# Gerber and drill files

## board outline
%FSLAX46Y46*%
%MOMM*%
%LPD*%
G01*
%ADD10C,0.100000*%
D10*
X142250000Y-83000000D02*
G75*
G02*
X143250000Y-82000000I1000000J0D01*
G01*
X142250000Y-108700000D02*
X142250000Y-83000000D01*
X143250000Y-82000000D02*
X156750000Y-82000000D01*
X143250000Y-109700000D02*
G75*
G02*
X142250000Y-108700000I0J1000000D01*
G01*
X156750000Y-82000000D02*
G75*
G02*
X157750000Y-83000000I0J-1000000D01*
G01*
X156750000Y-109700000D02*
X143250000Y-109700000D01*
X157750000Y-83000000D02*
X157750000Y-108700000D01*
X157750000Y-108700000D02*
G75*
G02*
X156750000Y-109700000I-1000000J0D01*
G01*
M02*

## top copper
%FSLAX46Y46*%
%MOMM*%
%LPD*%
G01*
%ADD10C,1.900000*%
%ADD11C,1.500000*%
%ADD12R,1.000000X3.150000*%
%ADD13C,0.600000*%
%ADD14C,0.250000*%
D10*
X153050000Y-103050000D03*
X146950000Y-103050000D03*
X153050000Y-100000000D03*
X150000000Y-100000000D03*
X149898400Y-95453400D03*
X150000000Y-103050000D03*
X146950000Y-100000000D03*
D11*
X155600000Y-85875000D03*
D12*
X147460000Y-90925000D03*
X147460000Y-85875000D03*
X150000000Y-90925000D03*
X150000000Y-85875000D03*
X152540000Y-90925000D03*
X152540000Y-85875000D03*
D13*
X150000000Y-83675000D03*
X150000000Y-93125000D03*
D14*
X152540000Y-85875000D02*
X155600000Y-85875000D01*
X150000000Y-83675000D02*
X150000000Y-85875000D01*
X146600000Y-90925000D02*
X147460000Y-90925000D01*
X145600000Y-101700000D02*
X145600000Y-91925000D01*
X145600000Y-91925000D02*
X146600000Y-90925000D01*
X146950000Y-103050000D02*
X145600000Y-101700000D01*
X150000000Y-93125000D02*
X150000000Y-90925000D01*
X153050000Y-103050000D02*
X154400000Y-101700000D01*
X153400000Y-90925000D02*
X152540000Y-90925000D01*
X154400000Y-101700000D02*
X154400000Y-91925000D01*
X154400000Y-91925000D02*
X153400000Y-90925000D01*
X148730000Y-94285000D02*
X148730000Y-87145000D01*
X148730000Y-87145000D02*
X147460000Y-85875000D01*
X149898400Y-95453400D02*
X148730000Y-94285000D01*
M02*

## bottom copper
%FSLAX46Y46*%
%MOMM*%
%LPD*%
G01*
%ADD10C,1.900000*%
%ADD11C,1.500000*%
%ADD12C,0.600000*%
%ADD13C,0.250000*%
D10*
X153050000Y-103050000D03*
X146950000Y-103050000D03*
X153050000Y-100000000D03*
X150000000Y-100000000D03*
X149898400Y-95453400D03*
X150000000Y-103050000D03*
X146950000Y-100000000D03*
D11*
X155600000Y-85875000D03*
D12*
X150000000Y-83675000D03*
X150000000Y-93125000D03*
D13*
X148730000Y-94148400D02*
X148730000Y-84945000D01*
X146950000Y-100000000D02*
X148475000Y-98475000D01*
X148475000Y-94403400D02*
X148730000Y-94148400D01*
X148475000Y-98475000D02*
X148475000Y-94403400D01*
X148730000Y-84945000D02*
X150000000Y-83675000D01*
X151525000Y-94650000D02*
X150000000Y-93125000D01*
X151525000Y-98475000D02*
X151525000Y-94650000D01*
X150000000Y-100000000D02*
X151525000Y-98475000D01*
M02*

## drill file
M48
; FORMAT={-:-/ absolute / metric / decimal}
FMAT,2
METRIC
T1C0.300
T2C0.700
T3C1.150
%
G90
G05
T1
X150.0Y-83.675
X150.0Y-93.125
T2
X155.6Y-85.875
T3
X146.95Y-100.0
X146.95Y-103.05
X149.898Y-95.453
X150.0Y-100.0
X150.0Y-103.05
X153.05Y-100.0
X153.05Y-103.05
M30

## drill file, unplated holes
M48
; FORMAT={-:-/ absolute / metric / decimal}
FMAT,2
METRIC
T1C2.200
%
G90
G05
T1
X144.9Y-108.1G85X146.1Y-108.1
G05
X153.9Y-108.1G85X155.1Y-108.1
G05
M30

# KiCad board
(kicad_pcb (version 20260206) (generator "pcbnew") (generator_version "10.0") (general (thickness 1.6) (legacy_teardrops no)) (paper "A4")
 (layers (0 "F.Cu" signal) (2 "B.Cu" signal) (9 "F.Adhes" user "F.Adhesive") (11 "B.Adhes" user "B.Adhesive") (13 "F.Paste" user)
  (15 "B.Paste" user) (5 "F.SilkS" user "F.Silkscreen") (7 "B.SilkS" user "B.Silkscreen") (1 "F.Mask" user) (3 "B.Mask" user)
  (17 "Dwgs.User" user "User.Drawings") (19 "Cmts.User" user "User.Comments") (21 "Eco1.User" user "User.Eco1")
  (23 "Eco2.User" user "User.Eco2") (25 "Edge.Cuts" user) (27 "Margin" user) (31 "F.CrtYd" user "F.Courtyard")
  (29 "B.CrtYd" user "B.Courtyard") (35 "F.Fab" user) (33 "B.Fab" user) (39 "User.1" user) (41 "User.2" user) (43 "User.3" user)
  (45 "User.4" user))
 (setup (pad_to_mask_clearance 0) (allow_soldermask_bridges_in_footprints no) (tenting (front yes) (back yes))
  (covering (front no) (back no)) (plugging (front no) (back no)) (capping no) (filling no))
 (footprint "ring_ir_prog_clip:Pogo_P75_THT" (layer "F.Cu") (at 153.05 103.05)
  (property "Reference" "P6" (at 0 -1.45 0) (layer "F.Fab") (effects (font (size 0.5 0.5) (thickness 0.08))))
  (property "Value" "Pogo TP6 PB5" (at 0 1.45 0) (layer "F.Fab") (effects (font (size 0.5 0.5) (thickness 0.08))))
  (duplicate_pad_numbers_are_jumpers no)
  (pad "1" thru_hole circle (at 0 0) (size 1.9 1.9) (drill 1.15) (layers "*.Cu" "*.Mask") (remove_unused_layers no) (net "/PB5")))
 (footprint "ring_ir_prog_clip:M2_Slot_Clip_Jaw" (layer "F.Cu") (at 154.5 108.1)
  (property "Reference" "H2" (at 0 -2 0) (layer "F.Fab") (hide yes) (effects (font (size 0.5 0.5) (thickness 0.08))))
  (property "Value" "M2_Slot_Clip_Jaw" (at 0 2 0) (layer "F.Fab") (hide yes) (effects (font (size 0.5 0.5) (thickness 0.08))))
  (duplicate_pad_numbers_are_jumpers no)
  (pad "" np_thru_hole oval (at 0 0) (size 3.4 2.2) (drill oval 3.4 2.2) (layers "*.Cu" "*.Mask")))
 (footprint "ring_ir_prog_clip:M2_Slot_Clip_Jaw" (layer "F.Cu") (at 145.5 108.1)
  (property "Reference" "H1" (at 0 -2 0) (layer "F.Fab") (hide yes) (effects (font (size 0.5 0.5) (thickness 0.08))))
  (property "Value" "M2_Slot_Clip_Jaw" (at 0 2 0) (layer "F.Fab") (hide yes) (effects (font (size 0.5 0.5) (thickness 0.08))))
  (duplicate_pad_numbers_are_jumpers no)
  (pad "" np_thru_hole oval (at 0 0) (size 3.4 2.2) (drill oval 3.4 2.2) (layers "*.Cu" "*.Mask")))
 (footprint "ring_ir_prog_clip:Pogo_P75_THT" (layer "F.Cu") (at 146.95 103.05)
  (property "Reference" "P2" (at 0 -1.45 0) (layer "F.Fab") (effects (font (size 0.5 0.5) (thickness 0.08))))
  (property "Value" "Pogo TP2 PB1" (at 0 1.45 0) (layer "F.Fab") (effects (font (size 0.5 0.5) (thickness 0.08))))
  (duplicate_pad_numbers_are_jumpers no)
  (pad "1" thru_hole circle (at 0 0) (size 1.9 1.9) (drill 1.15) (layers "*.Cu" "*.Mask") (remove_unused_layers no) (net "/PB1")))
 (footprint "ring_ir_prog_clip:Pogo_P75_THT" (layer "F.Cu") (at 153.05 100)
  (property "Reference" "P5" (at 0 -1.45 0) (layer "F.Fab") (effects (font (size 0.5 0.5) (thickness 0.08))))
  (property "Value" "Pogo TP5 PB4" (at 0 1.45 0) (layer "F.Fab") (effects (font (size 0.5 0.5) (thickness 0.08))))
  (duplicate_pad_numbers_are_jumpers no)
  (pad "1" thru_hole circle (at 0 0) (size 1.9 1.9) (drill 1.15) (layers "*.Cu" "*.Mask") (remove_unused_layers no)
   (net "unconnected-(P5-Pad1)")))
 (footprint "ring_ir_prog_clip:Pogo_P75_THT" (layer "F.Cu") (at 150 100)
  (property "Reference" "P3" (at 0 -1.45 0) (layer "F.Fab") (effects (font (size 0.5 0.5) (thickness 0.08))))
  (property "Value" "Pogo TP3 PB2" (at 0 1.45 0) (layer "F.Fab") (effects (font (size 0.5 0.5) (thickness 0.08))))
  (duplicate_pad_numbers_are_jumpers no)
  (pad "1" thru_hole circle (at 0 0) (size 1.9 1.9) (drill 1.15) (layers "*.Cu" "*.Mask") (remove_unused_layers no) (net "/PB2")))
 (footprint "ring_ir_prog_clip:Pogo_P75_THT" (layer "F.Cu") (at 149.8984 95.4534)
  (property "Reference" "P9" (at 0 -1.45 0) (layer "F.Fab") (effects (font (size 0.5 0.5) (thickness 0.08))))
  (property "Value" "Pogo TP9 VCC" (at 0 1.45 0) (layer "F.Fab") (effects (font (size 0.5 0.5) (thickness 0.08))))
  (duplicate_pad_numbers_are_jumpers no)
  (pad "1" thru_hole circle (at 0 0) (size 1.9 1.9) (drill 1.15) (layers "*.Cu" "*.Mask") (remove_unused_layers no) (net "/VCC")))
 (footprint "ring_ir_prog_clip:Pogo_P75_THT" (layer "F.Cu") (at 150 103.05)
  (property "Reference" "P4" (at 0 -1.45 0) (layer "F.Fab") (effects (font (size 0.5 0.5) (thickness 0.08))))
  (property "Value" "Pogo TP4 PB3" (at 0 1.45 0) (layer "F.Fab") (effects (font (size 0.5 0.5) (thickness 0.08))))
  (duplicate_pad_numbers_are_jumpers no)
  (pad "1" thru_hole circle (at 0 0) (size 1.9 1.9) (drill 1.15) (layers "*.Cu" "*.Mask") (remove_unused_layers no)
   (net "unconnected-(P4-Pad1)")))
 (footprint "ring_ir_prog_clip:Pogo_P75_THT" (layer "F.Cu") (at 146.95 100)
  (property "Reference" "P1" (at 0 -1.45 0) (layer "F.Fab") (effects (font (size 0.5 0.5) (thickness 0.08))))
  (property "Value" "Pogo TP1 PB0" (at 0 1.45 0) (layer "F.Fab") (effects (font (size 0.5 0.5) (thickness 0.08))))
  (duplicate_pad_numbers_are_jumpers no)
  (pad "1" thru_hole circle (at 0 0) (size 1.9 1.9) (drill 1.15) (layers "*.Cu" "*.Mask") (remove_unused_layers no) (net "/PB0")))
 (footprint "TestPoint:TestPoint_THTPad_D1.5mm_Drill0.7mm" (layer "F.Cu") (at 155.6 85.875)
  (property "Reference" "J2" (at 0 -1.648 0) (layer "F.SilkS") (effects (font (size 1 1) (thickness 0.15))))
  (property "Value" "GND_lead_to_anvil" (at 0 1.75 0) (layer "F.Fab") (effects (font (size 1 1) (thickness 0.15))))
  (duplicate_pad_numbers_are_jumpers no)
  (pad "1" thru_hole circle (at 0 0) (size 1.5 1.5) (drill 0.7) (layers "*.Cu" "*.Mask") (remove_unused_layers no) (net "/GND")))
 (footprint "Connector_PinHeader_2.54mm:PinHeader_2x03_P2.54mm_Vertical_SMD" (layer "F.Cu") (at 150 88.4 90)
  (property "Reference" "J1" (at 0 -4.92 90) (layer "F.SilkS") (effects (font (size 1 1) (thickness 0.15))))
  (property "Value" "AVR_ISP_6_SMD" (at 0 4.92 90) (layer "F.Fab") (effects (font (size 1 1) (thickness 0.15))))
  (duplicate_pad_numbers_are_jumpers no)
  (pad "1" smd rect (at -2.525 -2.54 90) (size 3.15 1) (layers "F.Cu" "F.Mask" "F.Paste") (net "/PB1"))
  (pad "2" smd rect (at 2.525 -2.54 90) (size 3.15 1) (layers "F.Cu" "F.Mask" "F.Paste") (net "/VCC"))
  (pad "3" smd rect (at -2.525 0 90) (size 3.15 1) (layers "F.Cu" "F.Mask" "F.Paste") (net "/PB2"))
  (pad "4" smd rect (at 2.525 0 90) (size 3.15 1) (layers "F.Cu" "F.Mask" "F.Paste") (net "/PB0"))
  (pad "5" smd rect (at -2.525 2.54 90) (size 3.15 1) (layers "F.Cu" "F.Mask" "F.Paste") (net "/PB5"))
  (pad "6" smd rect (at 2.525 2.54 90) (size 3.15 1) (layers "F.Cu" "F.Mask" "F.Paste") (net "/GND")))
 (gr_arc (start 142.25 83) (mid 142.542893 82.292893) (end 143.25 82) (stroke (width 0.1) (type default)) (layer "Edge.Cuts"))
 (gr_line (start 142.25 108.7) (end 142.25 83) (stroke (width 0.1) (type default)) (layer "Edge.Cuts"))
 (gr_line (start 143.25 82) (end 156.75 82) (stroke (width 0.1) (type default)) (layer "Edge.Cuts"))
 (gr_arc (start 143.25 109.7) (mid 142.542893 109.407106) (end 142.25 108.7) (stroke (width 0.1) (type default)) (layer "Edge.Cuts"))
 (gr_arc (start 156.75 82) (mid 157.457106 82.292893) (end 157.75 83) (stroke (width 0.1) (type default)) (layer "Edge.Cuts"))
 (gr_line (start 156.75 109.7) (end 143.25 109.7) (stroke (width 0.1) (type default)) (layer "Edge.Cuts"))
 (gr_line (start 157.75 83) (end 157.75 108.7) (stroke (width 0.1) (type default)) (layer "Edge.Cuts"))
 (gr_arc (start 157.75 108.7) (mid 157.457106 109.407106) (end 156.75 109.7) (stroke (width 0.1) (type default)) (layer "Edge.Cuts"))
 (segment (start 152.54 85.875) (end 155.6 85.875) (width 0.25) (layer "F.Cu") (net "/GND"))
 (segment (start 150 83.675) (end 150 85.875) (width 0.25) (layer "F.Cu") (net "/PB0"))
 (via (at 150 83.675) (size 0.6) (drill 0.3) (layers "F.Cu" "B.Cu") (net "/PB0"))
 (segment (start 148.73 94.1484) (end 148.73 84.945) (width 0.25) (layer "B.Cu") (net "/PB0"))
 (segment (start 146.95 100) (end 148.475 98.475) (width 0.25) (layer "B.Cu") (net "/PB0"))
 (segment (start 148.475 94.4034) (end 148.73 94.1484) (width 0.25) (layer "B.Cu") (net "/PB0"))
 (segment (start 148.475 98.475) (end 148.475 94.4034) (width 0.25) (layer "B.Cu") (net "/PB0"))
 (segment (start 148.73 84.945) (end 150 83.675) (width 0.25) (layer "B.Cu") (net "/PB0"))
 (segment (start 146.6 90.925) (end 147.46 90.925) (width 0.25) (layer "F.Cu") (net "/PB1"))
 (segment (start 145.6 101.7) (end 145.6 91.925) (width 0.25) (layer "F.Cu") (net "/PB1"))
 (segment (start 145.6 91.925) (end 146.6 90.925) (width 0.25) (layer "F.Cu") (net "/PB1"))
 (segment (start 146.95 103.05) (end 145.6 101.7) (width 0.25) (layer "F.Cu") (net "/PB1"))
 (segment (start 150 93.125) (end 150 90.925) (width 0.25) (layer "F.Cu") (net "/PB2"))
 (via (at 150 93.125) (size 0.6) (drill 0.3) (layers "F.Cu" "B.Cu") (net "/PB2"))
 (segment (start 151.525 94.65) (end 150 93.125) (width 0.25) (layer "B.Cu") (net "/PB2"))
 (segment (start 151.525 98.475) (end 151.525 94.65) (width 0.25) (layer "B.Cu") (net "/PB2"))
 (segment (start 150 100) (end 151.525 98.475) (width 0.25) (layer "B.Cu") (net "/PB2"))
 (segment (start 153.05 103.05) (end 154.4 101.7) (width 0.25) (layer "F.Cu") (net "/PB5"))
 (segment (start 153.4 90.925) (end 152.54 90.925) (width 0.25) (layer "F.Cu") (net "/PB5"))
 (segment (start 154.4 101.7) (end 154.4 91.925) (width 0.25) (layer "F.Cu") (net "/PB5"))
 (segment (start 154.4 91.925) (end 153.4 90.925) (width 0.25) (layer "F.Cu") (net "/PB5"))
 (segment (start 148.73 94.285) (end 148.73 87.145) (width 0.25) (layer "F.Cu") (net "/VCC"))
 (segment (start 148.73 87.145) (end 147.46 85.875) (width 0.25) (layer "F.Cu") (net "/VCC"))
 (segment (start 149.8984 95.4534) (end 148.73 94.285) (width 0.25) (layer "F.Cu") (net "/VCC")))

